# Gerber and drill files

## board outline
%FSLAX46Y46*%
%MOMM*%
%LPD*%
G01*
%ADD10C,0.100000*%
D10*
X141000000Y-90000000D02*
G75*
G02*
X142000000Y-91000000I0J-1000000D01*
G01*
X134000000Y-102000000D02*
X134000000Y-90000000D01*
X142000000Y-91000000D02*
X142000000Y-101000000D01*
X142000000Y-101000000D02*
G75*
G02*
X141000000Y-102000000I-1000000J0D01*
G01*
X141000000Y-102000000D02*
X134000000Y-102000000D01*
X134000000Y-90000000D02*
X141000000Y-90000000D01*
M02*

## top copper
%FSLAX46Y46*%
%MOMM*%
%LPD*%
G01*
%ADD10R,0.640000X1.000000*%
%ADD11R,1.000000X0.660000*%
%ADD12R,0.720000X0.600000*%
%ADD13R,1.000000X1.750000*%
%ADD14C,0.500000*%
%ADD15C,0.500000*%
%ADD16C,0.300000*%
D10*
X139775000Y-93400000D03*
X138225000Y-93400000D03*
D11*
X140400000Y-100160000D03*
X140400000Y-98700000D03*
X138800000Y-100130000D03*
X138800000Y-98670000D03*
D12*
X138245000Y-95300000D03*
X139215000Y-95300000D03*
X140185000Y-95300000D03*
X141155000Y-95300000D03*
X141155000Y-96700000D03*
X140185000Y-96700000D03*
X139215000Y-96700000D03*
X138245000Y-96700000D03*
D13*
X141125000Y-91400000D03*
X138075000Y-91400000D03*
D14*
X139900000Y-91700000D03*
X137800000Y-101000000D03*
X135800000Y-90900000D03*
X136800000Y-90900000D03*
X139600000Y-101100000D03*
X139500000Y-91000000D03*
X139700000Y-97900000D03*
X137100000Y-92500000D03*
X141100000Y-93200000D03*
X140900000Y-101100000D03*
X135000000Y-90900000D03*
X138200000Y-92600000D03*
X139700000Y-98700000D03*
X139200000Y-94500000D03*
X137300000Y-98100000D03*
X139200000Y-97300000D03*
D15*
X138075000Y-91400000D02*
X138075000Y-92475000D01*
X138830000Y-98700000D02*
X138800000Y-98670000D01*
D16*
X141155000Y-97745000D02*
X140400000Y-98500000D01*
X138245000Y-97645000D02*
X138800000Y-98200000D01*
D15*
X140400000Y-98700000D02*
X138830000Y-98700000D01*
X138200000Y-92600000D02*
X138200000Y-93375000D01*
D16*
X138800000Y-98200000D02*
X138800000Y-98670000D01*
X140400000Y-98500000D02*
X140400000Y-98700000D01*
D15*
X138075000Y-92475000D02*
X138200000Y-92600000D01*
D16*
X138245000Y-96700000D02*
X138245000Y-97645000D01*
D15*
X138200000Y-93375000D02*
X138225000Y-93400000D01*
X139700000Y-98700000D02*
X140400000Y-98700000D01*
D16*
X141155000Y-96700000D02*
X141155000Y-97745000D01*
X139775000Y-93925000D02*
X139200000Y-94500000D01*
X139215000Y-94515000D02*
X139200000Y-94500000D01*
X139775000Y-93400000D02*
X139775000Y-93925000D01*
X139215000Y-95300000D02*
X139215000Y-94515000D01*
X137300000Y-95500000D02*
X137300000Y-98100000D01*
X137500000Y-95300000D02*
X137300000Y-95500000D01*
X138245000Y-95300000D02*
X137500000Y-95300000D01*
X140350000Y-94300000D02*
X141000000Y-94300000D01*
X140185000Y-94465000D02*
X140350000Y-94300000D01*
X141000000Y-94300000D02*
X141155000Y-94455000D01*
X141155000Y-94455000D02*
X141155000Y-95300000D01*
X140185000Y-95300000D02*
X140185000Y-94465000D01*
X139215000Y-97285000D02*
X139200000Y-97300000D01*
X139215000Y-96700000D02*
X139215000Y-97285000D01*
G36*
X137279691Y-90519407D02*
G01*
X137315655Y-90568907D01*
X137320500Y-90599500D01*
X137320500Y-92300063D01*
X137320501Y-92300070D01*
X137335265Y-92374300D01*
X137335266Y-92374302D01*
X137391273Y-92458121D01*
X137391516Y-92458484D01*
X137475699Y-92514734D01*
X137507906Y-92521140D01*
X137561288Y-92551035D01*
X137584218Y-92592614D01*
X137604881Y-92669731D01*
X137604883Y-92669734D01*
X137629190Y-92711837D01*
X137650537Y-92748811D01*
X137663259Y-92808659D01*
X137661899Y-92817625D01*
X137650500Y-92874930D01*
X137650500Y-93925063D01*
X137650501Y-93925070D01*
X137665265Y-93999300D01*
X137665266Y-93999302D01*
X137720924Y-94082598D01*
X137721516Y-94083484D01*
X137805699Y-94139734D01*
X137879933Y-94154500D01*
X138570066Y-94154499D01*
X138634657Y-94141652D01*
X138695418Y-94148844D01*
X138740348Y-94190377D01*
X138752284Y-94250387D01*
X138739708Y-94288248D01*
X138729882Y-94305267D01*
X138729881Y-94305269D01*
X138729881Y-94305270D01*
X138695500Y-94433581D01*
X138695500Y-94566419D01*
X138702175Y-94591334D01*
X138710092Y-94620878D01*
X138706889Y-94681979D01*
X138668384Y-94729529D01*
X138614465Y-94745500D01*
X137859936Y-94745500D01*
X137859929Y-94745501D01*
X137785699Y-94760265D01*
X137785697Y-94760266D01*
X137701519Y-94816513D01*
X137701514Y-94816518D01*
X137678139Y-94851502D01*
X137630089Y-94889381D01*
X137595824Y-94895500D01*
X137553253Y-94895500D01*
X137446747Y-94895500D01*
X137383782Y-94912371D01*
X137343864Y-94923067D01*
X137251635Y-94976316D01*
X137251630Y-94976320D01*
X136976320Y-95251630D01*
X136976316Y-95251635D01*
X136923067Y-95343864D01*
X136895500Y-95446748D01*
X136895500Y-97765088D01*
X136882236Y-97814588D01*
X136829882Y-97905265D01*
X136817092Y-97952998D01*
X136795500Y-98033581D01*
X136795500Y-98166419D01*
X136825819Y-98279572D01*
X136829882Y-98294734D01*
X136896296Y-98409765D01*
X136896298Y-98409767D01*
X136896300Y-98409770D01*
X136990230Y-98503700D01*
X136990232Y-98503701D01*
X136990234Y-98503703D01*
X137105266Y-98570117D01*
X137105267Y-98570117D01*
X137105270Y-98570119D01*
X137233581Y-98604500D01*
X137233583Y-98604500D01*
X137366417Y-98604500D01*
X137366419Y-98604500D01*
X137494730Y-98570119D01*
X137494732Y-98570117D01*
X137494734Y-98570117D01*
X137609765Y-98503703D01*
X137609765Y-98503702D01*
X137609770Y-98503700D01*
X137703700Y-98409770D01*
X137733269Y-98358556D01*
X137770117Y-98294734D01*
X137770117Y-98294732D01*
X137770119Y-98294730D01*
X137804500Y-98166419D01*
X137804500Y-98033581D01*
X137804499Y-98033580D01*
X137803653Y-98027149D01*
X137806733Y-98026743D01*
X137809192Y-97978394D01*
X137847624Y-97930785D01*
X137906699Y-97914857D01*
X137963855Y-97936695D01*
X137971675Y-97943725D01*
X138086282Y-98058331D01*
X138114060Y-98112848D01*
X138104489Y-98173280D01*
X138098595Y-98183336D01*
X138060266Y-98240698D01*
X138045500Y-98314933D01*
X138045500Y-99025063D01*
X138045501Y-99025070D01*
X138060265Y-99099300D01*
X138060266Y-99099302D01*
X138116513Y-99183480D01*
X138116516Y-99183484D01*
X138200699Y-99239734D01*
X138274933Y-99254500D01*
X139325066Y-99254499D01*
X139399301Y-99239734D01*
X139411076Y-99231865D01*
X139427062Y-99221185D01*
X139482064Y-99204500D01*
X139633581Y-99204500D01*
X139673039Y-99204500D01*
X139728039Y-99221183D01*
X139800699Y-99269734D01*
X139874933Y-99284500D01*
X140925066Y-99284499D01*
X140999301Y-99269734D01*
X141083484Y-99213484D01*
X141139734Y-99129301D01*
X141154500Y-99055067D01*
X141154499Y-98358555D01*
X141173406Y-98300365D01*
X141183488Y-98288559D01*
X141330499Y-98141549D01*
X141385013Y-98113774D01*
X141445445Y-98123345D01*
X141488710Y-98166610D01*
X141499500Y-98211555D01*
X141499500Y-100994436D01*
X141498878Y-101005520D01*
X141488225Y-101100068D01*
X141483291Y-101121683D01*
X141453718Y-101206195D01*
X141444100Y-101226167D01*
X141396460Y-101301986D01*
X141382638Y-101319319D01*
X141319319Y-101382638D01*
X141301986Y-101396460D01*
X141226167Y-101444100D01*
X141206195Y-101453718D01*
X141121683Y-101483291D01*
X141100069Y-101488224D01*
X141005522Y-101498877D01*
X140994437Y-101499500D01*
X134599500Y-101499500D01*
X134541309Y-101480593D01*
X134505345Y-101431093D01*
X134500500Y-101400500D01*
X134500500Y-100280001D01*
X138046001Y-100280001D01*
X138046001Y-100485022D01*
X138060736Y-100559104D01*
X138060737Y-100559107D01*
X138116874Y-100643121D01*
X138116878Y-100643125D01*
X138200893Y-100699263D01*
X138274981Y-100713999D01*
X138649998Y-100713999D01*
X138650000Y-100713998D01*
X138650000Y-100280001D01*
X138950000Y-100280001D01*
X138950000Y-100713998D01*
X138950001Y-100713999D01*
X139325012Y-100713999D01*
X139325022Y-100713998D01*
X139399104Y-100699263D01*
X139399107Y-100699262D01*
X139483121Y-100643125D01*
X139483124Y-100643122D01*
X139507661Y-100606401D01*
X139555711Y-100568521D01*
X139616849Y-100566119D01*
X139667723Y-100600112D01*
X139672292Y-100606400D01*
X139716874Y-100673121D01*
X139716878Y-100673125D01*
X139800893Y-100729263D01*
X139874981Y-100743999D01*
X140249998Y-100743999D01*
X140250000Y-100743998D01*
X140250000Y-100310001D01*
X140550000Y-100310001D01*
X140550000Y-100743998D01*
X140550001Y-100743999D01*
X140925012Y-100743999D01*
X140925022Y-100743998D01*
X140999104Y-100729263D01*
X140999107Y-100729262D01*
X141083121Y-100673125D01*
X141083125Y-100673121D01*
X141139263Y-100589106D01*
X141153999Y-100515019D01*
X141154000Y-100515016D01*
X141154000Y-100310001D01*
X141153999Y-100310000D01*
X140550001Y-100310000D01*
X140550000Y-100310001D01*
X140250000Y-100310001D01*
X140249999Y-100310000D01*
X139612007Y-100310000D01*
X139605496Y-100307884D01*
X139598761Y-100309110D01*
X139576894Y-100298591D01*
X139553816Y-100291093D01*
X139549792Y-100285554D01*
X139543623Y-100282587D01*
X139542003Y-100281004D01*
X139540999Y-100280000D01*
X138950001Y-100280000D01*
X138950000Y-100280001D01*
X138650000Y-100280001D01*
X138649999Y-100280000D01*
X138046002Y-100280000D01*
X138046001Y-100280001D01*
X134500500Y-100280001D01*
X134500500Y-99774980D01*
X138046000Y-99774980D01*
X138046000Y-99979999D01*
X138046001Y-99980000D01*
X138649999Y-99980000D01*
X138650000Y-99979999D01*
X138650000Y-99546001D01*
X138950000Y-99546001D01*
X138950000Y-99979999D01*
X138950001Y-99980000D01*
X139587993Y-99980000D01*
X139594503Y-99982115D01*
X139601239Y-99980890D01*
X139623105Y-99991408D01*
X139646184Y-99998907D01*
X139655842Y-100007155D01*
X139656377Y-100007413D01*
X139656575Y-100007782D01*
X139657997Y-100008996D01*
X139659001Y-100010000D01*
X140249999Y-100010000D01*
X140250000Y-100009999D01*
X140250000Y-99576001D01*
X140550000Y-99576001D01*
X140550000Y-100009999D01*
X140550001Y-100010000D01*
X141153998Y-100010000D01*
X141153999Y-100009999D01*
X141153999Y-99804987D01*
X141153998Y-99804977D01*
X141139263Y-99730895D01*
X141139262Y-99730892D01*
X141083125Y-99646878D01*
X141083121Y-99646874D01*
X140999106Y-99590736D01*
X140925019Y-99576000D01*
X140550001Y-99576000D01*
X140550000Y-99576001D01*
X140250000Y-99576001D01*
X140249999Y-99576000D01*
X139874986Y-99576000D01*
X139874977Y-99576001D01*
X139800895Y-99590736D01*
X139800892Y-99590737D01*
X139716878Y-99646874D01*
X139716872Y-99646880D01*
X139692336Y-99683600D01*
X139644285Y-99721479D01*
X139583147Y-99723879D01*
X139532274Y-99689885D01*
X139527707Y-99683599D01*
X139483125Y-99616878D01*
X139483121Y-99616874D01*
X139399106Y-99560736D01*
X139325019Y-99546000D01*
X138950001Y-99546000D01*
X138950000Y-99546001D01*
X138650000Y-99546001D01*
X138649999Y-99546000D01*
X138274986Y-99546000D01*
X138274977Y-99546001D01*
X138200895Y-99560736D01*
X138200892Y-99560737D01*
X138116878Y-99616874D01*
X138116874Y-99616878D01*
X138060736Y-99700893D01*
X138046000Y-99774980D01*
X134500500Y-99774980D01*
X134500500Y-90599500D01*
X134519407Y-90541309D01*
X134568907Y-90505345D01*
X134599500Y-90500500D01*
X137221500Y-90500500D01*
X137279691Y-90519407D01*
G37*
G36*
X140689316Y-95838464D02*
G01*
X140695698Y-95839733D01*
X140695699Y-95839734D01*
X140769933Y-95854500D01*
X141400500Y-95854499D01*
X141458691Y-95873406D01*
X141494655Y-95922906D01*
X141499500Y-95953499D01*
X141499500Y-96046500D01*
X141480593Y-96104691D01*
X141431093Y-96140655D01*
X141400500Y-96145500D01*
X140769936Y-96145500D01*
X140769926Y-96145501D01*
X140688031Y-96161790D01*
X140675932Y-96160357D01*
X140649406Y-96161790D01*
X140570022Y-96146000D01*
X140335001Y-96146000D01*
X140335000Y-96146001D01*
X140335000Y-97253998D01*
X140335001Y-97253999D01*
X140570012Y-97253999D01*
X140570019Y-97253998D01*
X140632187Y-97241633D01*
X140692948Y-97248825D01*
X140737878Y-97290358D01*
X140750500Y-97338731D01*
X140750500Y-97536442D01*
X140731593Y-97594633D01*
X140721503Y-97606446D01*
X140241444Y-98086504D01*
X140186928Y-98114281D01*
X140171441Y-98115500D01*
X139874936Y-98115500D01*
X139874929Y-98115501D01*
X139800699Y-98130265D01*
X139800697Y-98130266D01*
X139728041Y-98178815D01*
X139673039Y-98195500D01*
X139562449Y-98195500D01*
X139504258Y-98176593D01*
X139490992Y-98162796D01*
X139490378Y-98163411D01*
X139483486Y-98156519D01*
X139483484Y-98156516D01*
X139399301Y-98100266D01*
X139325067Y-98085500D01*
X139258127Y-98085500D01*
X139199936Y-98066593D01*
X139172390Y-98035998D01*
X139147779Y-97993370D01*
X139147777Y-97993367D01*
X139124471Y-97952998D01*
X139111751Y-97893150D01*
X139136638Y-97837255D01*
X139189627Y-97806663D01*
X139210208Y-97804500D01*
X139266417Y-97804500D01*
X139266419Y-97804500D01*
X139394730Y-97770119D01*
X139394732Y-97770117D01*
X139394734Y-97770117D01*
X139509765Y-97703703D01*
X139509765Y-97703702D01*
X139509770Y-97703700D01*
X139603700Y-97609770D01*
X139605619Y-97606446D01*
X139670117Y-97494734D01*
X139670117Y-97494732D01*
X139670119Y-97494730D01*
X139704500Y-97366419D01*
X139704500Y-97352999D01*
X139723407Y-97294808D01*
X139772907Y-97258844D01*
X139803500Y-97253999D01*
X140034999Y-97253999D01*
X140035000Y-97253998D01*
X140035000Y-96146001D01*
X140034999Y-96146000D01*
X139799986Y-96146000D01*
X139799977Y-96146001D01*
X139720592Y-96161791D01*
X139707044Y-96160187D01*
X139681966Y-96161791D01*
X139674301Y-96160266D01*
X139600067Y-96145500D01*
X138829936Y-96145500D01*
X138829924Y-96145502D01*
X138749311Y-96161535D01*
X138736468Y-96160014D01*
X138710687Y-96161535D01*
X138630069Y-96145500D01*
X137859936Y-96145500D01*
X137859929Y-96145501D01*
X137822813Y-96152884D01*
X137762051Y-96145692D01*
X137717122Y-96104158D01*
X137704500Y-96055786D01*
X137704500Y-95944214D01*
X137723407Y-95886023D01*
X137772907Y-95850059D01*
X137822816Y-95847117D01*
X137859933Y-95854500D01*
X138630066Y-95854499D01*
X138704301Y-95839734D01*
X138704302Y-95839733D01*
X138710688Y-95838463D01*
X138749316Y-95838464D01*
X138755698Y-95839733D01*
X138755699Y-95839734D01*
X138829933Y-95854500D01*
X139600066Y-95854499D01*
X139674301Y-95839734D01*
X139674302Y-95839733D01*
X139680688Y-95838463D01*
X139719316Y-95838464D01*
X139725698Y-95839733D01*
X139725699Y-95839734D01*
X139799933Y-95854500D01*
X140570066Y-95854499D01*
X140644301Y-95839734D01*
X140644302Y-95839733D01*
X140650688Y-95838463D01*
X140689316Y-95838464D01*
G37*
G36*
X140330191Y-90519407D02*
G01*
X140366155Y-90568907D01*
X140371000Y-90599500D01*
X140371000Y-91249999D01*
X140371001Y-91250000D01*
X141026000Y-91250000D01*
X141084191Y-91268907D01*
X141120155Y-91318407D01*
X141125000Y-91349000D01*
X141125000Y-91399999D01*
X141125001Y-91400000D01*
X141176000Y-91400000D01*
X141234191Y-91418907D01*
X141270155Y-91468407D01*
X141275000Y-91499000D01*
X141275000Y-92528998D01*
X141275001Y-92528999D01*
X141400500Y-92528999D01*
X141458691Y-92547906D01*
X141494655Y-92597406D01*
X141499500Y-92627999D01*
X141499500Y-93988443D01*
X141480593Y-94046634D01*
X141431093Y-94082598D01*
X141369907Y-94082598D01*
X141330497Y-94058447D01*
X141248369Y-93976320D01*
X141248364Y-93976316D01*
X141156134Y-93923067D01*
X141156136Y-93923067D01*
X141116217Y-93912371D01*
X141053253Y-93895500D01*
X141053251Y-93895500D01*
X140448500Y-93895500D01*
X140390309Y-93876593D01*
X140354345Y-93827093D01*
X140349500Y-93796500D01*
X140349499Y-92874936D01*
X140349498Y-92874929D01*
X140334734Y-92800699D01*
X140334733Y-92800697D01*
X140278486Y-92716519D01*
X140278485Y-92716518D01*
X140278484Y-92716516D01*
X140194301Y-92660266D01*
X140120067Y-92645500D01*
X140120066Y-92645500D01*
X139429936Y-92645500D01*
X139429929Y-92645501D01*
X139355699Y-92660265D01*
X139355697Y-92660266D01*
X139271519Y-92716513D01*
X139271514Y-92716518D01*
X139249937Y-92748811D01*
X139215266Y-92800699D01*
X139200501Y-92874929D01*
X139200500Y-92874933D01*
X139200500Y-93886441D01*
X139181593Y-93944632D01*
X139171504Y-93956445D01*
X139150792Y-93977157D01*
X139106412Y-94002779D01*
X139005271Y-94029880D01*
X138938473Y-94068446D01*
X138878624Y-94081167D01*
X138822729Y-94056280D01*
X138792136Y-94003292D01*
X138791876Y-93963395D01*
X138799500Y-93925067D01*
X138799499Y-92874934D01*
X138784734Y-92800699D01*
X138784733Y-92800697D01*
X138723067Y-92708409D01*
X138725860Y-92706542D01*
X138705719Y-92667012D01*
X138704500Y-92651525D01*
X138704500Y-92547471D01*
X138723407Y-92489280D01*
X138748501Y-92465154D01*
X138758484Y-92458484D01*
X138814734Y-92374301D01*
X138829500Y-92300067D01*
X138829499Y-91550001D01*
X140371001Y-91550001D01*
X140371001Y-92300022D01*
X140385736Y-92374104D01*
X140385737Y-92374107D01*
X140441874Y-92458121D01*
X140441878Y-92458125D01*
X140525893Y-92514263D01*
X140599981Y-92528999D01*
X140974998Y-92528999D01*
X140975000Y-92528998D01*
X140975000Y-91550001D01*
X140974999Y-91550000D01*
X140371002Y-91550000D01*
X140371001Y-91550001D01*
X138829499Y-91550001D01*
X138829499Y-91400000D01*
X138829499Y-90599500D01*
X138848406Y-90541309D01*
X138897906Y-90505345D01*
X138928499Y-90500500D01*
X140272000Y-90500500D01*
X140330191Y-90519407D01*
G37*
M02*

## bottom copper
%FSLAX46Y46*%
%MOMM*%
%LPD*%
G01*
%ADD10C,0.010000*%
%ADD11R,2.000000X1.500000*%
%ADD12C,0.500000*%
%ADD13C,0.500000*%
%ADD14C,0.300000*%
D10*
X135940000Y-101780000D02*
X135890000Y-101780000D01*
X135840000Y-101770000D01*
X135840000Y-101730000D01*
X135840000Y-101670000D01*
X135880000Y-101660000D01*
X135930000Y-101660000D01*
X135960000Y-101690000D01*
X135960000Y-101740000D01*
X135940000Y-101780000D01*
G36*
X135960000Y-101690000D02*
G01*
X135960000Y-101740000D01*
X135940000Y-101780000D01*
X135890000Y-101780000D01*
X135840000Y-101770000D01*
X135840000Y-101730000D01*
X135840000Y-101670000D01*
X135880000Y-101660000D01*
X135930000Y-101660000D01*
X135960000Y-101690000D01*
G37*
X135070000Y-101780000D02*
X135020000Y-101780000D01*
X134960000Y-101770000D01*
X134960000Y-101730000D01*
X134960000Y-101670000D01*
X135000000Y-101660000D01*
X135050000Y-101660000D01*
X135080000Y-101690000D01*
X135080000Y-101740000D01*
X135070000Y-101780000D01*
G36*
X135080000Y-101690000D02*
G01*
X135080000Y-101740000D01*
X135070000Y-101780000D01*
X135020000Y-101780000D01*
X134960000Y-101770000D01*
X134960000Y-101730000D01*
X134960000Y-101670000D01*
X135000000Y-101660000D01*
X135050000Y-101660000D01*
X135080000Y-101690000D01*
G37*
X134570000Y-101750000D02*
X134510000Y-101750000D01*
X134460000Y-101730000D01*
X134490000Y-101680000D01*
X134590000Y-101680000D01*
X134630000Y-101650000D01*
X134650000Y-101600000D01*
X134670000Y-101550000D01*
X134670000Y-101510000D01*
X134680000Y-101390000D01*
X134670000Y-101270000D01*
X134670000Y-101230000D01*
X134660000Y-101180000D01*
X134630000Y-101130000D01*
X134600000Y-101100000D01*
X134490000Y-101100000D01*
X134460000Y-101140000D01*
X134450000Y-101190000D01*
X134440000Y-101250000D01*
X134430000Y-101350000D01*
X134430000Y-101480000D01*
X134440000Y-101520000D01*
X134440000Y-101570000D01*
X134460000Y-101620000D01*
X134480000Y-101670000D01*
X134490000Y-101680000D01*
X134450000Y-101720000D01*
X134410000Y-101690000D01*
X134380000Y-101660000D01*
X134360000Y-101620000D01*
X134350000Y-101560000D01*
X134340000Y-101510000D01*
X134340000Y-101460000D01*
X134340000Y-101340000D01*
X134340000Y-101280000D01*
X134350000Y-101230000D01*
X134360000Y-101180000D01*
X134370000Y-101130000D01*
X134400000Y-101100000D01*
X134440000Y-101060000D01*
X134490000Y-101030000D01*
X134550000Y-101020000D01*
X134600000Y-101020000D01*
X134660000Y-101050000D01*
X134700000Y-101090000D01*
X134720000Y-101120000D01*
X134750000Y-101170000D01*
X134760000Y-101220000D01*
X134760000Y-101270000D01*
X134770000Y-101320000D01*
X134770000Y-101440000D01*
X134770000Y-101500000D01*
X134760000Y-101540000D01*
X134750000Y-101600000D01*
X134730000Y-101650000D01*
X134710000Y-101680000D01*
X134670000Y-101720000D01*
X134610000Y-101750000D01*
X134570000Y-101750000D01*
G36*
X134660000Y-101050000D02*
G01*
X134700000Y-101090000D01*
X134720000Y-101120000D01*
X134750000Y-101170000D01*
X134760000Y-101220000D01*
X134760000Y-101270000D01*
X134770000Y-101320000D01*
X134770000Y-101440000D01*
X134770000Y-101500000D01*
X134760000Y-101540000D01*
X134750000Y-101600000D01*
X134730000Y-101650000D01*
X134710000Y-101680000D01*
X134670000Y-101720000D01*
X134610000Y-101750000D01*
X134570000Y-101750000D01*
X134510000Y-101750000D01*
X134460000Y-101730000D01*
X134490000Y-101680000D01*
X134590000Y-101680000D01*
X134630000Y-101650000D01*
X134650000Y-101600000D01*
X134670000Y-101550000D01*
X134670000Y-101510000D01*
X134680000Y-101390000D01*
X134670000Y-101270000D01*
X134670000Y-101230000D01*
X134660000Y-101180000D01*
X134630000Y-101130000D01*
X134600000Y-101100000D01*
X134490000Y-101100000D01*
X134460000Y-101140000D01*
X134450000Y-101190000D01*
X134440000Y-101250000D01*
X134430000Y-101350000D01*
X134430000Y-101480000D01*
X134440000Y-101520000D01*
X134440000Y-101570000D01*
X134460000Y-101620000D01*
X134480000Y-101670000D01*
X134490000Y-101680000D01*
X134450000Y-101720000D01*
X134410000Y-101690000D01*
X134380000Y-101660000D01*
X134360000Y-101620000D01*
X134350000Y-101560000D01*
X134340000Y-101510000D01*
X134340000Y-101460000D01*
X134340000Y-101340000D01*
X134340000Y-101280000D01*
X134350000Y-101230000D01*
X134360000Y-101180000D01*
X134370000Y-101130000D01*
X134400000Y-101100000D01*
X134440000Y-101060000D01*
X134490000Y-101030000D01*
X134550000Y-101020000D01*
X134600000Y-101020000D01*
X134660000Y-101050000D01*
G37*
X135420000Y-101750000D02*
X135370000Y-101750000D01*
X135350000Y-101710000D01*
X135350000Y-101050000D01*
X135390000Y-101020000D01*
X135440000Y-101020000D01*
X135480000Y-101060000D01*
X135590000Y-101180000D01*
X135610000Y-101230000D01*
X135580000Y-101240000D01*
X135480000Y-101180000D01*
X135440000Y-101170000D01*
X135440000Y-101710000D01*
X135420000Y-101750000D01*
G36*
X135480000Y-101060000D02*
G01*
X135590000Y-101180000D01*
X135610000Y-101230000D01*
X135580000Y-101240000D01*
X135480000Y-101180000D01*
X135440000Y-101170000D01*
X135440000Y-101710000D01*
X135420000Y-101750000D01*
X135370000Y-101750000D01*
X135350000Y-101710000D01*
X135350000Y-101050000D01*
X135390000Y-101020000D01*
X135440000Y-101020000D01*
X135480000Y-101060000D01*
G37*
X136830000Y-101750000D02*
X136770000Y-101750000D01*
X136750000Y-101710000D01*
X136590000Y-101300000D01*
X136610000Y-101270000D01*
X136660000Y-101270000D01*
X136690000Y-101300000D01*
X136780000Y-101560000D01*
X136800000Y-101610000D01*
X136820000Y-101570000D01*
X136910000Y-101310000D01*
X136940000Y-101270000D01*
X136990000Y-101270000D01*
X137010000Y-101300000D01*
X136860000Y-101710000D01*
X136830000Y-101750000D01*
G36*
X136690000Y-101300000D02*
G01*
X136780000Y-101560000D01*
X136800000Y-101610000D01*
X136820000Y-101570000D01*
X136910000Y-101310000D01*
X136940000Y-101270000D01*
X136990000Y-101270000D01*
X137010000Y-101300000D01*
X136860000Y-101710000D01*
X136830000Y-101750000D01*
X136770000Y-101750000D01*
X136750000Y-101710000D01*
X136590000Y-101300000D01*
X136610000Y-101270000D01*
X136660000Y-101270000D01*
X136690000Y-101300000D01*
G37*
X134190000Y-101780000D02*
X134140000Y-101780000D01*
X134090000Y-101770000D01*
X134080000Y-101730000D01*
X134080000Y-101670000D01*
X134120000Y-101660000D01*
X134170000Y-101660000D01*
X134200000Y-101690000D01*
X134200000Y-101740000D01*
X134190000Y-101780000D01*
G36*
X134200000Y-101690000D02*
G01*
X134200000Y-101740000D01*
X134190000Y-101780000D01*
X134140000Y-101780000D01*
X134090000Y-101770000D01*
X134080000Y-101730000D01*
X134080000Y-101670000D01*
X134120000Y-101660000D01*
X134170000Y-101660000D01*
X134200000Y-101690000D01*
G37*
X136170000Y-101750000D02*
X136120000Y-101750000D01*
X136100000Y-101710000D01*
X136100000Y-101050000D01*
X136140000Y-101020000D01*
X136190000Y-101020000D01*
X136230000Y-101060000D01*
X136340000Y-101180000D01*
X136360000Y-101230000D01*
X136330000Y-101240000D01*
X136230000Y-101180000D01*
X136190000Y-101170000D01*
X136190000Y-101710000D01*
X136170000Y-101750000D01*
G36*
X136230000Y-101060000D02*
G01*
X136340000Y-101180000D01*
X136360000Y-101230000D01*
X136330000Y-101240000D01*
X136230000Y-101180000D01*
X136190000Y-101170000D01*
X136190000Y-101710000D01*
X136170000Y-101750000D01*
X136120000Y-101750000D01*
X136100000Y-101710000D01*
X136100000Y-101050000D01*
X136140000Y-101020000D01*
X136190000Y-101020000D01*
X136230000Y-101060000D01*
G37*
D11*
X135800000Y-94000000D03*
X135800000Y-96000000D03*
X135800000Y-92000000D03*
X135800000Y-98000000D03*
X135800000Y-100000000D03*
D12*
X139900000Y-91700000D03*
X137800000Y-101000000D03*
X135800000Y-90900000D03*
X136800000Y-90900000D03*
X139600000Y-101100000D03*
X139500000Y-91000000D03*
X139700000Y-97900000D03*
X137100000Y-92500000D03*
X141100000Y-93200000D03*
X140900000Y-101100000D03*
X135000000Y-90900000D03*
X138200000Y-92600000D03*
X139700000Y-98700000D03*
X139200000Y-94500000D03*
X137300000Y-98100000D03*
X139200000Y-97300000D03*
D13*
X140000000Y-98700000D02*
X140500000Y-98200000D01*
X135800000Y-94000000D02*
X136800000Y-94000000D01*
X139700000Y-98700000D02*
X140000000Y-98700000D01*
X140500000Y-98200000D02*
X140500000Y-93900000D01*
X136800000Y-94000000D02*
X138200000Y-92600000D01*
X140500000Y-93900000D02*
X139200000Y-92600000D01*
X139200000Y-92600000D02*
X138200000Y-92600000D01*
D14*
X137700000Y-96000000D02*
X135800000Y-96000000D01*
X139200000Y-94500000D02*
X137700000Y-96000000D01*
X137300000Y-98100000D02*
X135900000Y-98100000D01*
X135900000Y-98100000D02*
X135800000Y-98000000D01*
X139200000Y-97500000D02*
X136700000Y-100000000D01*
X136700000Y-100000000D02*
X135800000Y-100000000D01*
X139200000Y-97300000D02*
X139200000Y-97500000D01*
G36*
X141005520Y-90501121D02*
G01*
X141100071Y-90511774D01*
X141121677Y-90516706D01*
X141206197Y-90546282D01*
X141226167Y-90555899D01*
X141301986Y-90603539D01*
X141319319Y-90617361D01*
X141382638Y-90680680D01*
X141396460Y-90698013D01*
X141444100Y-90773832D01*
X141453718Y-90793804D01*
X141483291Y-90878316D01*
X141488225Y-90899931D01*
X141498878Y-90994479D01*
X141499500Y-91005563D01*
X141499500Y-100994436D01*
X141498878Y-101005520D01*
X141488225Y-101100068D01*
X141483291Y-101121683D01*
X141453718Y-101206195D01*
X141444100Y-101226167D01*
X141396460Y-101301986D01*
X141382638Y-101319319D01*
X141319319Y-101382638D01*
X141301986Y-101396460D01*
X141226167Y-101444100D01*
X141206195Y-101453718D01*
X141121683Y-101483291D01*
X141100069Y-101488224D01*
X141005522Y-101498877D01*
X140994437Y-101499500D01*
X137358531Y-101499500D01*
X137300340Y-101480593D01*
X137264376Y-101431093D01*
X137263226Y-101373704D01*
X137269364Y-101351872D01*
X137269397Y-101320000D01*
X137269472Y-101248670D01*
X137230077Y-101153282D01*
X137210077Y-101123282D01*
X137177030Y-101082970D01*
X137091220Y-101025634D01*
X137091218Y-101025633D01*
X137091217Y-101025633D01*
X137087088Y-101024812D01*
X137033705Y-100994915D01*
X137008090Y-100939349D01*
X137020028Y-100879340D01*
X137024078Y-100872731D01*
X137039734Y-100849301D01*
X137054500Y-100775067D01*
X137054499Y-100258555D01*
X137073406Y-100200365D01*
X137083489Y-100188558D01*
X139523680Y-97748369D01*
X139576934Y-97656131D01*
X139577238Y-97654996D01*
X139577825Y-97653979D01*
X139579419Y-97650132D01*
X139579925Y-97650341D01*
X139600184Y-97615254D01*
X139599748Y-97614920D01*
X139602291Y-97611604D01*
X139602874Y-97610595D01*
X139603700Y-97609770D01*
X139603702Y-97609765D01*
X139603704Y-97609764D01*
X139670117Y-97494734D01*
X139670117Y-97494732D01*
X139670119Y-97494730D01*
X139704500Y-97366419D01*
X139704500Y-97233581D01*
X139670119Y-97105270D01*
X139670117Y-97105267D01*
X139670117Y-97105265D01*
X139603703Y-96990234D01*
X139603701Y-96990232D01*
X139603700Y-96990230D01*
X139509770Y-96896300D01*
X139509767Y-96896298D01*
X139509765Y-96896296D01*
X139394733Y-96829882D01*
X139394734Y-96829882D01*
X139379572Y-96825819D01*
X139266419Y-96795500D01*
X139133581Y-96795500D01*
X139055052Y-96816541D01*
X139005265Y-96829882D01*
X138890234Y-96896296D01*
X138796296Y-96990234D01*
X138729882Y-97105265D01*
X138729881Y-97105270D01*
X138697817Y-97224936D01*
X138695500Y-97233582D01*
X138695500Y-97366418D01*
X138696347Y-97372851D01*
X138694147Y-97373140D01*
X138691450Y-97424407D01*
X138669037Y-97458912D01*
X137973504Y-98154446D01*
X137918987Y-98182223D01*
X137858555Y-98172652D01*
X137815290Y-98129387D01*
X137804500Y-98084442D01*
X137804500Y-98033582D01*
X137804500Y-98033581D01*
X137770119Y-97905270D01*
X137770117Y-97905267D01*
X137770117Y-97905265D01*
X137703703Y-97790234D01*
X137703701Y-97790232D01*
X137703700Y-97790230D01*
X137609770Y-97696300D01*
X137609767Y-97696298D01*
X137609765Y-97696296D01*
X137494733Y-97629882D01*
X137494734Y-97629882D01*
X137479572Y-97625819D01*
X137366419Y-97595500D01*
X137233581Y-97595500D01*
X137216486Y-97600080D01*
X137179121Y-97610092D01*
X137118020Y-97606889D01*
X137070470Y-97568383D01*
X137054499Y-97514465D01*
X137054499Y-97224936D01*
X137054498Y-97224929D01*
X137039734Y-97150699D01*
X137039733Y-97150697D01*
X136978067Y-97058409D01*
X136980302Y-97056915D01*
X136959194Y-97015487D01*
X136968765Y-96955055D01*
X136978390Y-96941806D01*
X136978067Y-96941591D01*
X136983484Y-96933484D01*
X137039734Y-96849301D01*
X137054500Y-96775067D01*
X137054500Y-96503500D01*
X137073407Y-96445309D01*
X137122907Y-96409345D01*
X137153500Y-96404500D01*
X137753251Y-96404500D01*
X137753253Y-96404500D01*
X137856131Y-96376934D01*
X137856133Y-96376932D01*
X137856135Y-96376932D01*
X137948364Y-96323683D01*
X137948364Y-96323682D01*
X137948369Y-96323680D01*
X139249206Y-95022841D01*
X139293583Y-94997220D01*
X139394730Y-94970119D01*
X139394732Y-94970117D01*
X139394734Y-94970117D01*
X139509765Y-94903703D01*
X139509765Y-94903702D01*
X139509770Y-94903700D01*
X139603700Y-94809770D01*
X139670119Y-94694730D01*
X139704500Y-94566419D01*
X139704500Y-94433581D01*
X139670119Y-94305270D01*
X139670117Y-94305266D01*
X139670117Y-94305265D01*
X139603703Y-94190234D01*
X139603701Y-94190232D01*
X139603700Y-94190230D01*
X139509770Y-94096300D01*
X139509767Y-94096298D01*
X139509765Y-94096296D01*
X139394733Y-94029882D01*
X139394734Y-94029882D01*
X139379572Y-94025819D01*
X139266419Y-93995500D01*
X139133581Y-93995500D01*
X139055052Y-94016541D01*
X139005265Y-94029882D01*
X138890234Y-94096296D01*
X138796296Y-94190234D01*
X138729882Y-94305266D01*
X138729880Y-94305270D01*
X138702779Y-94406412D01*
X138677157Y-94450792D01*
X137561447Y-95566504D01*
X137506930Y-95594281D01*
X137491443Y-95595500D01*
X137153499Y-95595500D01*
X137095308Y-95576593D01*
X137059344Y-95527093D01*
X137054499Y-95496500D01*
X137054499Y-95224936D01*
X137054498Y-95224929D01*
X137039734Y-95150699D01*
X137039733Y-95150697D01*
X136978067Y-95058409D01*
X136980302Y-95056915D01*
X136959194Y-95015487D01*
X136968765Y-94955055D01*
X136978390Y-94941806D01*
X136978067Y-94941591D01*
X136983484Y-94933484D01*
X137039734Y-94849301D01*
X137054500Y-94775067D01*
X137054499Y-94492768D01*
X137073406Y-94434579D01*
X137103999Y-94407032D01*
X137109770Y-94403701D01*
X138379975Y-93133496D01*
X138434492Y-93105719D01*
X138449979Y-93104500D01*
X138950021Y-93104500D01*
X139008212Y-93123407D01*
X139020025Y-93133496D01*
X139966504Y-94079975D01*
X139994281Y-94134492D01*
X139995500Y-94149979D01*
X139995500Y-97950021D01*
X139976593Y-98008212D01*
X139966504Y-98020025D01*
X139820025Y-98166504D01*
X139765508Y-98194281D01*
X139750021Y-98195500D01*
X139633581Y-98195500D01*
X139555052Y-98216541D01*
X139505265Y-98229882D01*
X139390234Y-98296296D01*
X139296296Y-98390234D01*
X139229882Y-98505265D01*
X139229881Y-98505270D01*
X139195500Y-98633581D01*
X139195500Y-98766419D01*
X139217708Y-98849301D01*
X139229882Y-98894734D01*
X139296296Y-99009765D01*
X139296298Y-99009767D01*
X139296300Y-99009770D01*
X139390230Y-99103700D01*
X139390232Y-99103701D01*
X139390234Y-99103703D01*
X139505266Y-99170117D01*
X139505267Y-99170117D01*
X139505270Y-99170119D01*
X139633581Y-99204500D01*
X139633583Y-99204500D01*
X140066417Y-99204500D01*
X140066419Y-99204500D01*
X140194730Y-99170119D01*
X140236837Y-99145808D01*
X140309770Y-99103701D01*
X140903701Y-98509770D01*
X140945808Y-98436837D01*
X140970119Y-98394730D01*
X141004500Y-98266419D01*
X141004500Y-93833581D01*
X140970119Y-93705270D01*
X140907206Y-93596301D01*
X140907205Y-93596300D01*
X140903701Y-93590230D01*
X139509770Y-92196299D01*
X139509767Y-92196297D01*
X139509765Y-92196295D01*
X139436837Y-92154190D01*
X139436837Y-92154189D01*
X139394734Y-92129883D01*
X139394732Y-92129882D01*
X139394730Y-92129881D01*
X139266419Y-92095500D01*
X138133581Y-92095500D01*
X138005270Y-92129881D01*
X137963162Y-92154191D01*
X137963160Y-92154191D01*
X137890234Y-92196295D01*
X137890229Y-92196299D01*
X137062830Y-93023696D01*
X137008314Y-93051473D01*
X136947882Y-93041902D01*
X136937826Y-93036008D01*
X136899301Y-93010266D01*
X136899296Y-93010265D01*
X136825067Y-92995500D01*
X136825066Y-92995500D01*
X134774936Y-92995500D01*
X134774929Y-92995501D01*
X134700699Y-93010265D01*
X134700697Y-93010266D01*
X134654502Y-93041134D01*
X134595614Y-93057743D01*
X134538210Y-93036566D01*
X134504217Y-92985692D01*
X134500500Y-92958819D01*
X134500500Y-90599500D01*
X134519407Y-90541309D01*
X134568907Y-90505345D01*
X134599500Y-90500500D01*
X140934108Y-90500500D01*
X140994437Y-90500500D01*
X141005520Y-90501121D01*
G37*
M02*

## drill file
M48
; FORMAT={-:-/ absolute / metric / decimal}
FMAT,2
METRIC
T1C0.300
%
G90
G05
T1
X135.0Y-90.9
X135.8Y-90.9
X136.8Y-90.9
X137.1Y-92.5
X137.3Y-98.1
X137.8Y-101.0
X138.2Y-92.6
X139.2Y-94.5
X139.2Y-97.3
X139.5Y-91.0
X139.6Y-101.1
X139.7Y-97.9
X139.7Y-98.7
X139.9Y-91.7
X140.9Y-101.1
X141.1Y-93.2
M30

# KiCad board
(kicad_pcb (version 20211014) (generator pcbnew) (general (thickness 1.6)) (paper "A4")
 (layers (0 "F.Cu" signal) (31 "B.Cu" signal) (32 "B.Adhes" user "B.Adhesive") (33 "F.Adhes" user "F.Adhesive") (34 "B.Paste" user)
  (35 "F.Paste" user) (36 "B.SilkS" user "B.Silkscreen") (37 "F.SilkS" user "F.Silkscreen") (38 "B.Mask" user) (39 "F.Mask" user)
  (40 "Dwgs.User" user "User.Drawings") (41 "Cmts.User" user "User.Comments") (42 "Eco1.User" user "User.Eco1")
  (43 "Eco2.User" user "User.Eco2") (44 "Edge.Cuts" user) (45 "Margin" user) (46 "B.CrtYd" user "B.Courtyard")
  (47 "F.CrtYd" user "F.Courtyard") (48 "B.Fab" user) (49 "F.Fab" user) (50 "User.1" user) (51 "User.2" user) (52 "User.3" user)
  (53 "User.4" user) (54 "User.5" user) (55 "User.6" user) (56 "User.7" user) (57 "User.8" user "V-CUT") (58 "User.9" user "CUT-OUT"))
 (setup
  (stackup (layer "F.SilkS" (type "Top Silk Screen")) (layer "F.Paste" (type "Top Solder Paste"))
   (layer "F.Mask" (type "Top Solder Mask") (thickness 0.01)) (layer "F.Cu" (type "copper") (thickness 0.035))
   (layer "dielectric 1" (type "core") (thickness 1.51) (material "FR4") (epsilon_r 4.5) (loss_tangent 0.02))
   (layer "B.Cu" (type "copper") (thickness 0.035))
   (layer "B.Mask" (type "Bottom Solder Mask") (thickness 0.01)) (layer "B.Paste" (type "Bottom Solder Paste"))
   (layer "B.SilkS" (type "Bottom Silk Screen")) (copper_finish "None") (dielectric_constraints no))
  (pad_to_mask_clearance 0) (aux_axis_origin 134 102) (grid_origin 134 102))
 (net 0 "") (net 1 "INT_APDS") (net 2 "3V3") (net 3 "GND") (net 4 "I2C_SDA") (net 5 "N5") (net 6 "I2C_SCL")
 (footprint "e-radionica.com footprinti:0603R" (layer "F.Cu") (at 139 93.4 180)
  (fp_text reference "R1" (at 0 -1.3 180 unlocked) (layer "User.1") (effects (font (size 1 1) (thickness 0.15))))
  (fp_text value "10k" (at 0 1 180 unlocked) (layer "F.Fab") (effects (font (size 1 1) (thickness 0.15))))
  (pad "1" smd rect locked (at -0.775 0 270) (size 1 0.64) (layers "F.Cu" "F.Paste" "F.Mask") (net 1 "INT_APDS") (solder_mask_margin 0.1))
  (pad "2" smd rect locked (at 0.775 0 270) (size 1 0.64) (layers "F.Cu" "F.Paste" "F.Mask") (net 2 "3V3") (solder_mask_margin 0.1)))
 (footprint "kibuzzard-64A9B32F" (layer "F.Cu") (at 135 96 -90)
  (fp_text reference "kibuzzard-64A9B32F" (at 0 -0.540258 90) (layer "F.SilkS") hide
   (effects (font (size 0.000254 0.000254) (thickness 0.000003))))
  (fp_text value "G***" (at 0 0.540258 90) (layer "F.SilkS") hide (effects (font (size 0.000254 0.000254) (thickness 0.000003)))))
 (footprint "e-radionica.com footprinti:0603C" (layer "F.Cu") (at 140.4 99.43 90)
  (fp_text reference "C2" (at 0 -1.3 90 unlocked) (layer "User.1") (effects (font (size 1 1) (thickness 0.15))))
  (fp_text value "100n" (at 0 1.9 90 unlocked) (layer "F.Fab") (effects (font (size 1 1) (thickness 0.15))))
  (pad "1" smd rect locked (at -0.73 0 90) (size 0.66 1) (layers "F.Cu" "F.Paste" "F.Mask") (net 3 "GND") (solder_mask_margin 0.1))
  (pad "2" smd rect locked (at 0.73 0 90) (size 0.66 1) (layers "F.Cu" "F.Paste" "F.Mask") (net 2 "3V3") (solder_mask_margin 0.1)))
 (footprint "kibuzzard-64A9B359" (layer "F.Cu") (at 136.5 96 -90)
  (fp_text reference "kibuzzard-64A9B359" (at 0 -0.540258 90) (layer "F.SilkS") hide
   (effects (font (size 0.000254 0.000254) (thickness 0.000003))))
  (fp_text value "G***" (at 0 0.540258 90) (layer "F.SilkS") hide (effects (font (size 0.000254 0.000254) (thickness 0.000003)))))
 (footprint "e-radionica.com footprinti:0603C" (layer "F.Cu") (at 138.8 99.4 90)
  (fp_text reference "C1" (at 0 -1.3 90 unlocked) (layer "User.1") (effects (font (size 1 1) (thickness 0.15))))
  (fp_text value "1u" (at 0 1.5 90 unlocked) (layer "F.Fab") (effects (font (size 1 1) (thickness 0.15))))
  (pad "1" smd rect locked (at -0.73 0 90) (size 0.66 1) (layers "F.Cu" "F.Paste" "F.Mask") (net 3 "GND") (solder_mask_margin 0.1))
  (pad "2" smd rect locked (at 0.73 0 90) (size 0.66 1) (layers "F.Cu" "F.Paste" "F.Mask") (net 2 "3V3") (solder_mask_margin 0.1)))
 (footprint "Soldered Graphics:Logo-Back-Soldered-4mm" (layer "F.Cu") (at 139.5 96 90)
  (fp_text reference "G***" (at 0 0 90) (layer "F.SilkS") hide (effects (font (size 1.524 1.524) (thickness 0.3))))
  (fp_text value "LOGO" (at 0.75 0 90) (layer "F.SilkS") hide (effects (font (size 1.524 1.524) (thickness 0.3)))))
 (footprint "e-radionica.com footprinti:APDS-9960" (layer "F.Cu") (at 139.7 96 90)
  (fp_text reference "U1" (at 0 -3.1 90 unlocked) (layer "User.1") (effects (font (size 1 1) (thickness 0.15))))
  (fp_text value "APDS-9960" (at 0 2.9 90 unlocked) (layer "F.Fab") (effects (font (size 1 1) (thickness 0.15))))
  (pad "1" smd rect (at 0.7 -1.455 90) (size 0.6 0.72) (layers "F.Cu" "F.Paste" "F.Mask") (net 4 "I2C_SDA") (solder_mask_margin 0.1))
  (pad "2" smd rect (at 0.7 -0.485 90) (size 0.6 0.72) (layers "F.Cu" "F.Paste" "F.Mask") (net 1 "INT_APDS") (solder_mask_margin 0.1))
  (pad "3" smd rect (at 0.7 0.485 90) (size 0.6 0.72) (layers "F.Cu" "F.Paste" "F.Mask") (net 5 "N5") (solder_mask_margin 0.1))
  (pad "4" smd rect (at 0.7 1.455 90) (size 0.6 0.72) (layers "F.Cu" "F.Paste" "F.Mask") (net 5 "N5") (solder_mask_margin 0.1))
  (pad "5" smd rect (at -0.7 1.455 90) (size 0.6 0.72) (layers "F.Cu" "F.Paste" "F.Mask") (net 2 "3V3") (solder_mask_margin 0.1))
  (pad "6" smd rect (at -0.7 0.485 90) (size 0.6 0.72) (layers "F.Cu" "F.Paste" "F.Mask") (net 3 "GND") (solder_mask_margin 0.1))
  (pad "7" smd rect (at -0.7 -0.485 90) (size 0.6 0.72) (layers "F.Cu" "F.Paste" "F.Mask") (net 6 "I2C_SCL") (solder_mask_margin 0.1))
  (pad "8" smd rect (at -0.7 -1.455 90) (size 0.6 0.72) (layers "F.Cu" "F.Paste" "F.Mask") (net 2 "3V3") (solder_mask_margin 0.1)))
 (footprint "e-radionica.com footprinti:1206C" (layer "F.Cu") (at 139.6 91.4 180)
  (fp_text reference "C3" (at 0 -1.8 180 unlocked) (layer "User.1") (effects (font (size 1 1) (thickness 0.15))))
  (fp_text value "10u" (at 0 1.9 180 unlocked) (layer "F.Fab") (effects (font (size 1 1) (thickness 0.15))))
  (pad "1" smd rect locked (at -1.525 0 270) (size 1.75 1) (layers "F.Cu" "F.Paste" "F.Mask") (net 3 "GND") (solder_mask_margin 0.1))
  (pad "2" smd rect locked (at 1.525 0 270) (size 1.75 1) (layers "F.Cu" "F.Paste" "F.Mask") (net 2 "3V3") (solder_mask_margin 0.1)))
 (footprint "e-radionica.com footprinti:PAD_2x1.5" (layer "B.Cu") (at 135.8 94 180)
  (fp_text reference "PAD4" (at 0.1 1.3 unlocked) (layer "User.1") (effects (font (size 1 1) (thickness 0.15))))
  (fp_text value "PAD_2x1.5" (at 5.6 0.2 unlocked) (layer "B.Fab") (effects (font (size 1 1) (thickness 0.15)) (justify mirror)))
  (pad "1" smd rect (at 0 0 180) (size 2 1.5) (layers "B.Cu" "B.Paste" "B.Mask") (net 2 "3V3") (solder_mask_margin 0.1)))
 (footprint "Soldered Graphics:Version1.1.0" (layer "B.Cu") (at 135.5 101.4 180)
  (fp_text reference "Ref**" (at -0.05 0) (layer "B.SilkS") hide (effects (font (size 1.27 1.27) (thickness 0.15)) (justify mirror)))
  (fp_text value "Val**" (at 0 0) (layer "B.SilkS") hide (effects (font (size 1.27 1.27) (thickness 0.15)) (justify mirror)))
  (fp_poly
   (pts (xy -0.44 -0.38) (xy -0.39 -0.38) (xy -0.34 -0.37) (xy -0.34 -0.33) (xy -0.34 -0.27) (xy -0.38 -0.26) (xy -0.43 -0.26)
    (xy -0.46 -0.29) (xy -0.46 -0.34) (xy -0.44 -0.38))
   (layer "B.Cu") (width 0.01) (fill solid))
  (fp_poly
   (pts (xy 0.43 -0.38) (xy 0.48 -0.38) (xy 0.54 -0.37) (xy 0.54 -0.33) (xy 0.54 -0.27) (xy 0.5 -0.26) (xy 0.45 -0.26) (xy 0.42 -0.29)
    (xy 0.42 -0.34) (xy 0.43 -0.38))
   (layer "B.Cu") (width 0.01) (fill solid))
  (fp_poly
   (pts (xy 0.93 -0.35) (xy 0.99 -0.35) (xy 1.04 -0.33) (xy 1.01 -0.28) (xy 0.91 -0.28) (xy 0.87 -0.25) (xy 0.85 -0.2) (xy 0.83 -0.15)
    (xy 0.83 -0.11) (xy 0.82 0.01) (xy 0.83 0.13) (xy 0.83 0.17) (xy 0.84 0.22) (xy 0.87 0.27) (xy 0.9 0.3) (xy 1.01 0.3) (xy 1.04 0.26)
    (xy 1.05 0.21) (xy 1.06 0.15) (xy 1.07 0.05) (xy 1.07 -0.08) (xy 1.06 -0.12) (xy 1.06 -0.17) (xy 1.04 -0.22) (xy 1.02 -0.27)
    (xy 1.01 -0.28) (xy 1.05 -0.32) (xy 1.09 -0.29) (xy 1.12 -0.26) (xy 1.14 -0.22) (xy 1.15 -0.16) (xy 1.16 -0.11) (xy 1.16 -0.06)
    (xy 1.16 0.06) (xy 1.16 0.12) (xy 1.15 0.17) (xy 1.14 0.22) (xy 1.13 0.27) (xy 1.1 0.3) (xy 1.06 0.34) (xy 1.01 0.37) (xy 0.95 0.38)
    (xy 0.9 0.38) (xy 0.84 0.35) (xy 0.8 0.31) (xy 0.78 0.28) (xy 0.75 0.23) (xy 0.74 0.18) (xy 0.74 0.13) (xy 0.73 0.08) (xy 0.73 -0.04)
    (xy 0.73 -0.1) (xy 0.74 -0.14) (xy 0.75 -0.2) (xy 0.77 -0.25) (xy 0.79 -0.28) (xy 0.83 -0.32) (xy 0.89 -0.35) (xy 0.93 -0.35))
   (layer "B.Cu") (width 0.01) (fill solid))
  (fp_poly
   (pts (xy 0.08 -0.35) (xy 0.13 -0.35) (xy 0.15 -0.31) (xy 0.15 0.35) (xy 0.11 0.38) (xy 0.06 0.38) (xy 0.02 0.34) (xy -0.09 0.22)
    (xy -0.11 0.17) (xy -0.08 0.16) (xy 0.02 0.22) (xy 0.06 0.23) (xy 0.06 -0.31) (xy 0.08 -0.35))
   (layer "B.Cu") (width 0.01) (fill solid))
  (fp_poly
   (pts (xy -1.33 -0.35) (xy -1.27 -0.35) (xy -1.25 -0.31) (xy -1.09 0.1) (xy -1.11 0.13) (xy -1.16 0.13) (xy -1.19 0.1) (xy -1.28 -0.16)
    (xy -1.3 -0.21) (xy -1.32 -0.17) (xy -1.41 0.09) (xy -1.44 0.13) (xy -1.49 0.13) (xy -1.51 0.1) (xy -1.36 -0.31) (xy -1.33 -0.35))
   (layer "B.Cu") (width 0.01) (fill solid))
  (fp_poly
   (pts (xy 1.31 -0.38) (xy 1.36 -0.38) (xy 1.41 -0.37) (xy 1.42 -0.33) (xy 1.42 -0.27) (xy 1.38 -0.26) (xy 1.33 -0.26) (xy 1.3 -0.29)
    (xy 1.3 -0.34) (xy 1.31 -0.38))
   (layer "B.Cu") (width 0.01) (fill solid))
  (fp_poly
   (pts (xy -0.67 -0.35) (xy -0.62 -0.35) (xy -0.6 -0.31) (xy -0.6 0.35) (xy -0.64 0.38) (xy -0.69 0.38) (xy -0.73 0.34) (xy -0.84 0.22)
    (xy -0.86 0.17) (xy -0.83 0.16) (xy -0.73 0.22) (xy -0.69 0.23) (xy -0.69 -0.31) (xy -0.67 -0.35))
   (layer "B.Cu") (width 0.01) (fill solid)))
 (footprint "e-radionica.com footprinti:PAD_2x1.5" (layer "B.Cu") (at 135.8 96 180)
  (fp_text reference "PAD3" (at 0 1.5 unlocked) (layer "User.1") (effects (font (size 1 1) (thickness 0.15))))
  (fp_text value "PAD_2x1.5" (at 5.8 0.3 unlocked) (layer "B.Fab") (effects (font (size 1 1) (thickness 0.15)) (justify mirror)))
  (pad "1" smd rect (at 0 0 180) (size 2 1.5) (layers "B.Cu" "B.Paste" "B.Mask") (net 1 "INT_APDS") (solder_mask_margin 0.1)))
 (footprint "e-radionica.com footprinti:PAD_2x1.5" (layer "B.Cu") (at 135.8 92 180)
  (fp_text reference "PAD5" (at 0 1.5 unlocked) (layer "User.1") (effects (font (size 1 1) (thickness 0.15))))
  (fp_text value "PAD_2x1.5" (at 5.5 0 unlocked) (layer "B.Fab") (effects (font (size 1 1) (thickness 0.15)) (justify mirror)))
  (pad "1" smd rect (at 0 0 180) (size 2 1.5) (layers "B.Cu" "B.Paste" "B.Mask") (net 3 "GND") (solder_mask_margin 0.1) (zone_connect 2)))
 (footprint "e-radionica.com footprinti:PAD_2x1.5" (layer "B.Cu") (at 135.8 98 180)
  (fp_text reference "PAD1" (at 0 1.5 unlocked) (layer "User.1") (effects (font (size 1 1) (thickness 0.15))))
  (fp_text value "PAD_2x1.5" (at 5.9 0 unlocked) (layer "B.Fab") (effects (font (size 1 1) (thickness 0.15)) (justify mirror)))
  (pad "1" smd rect (at 0 0 180) (size 2 1.5) (layers "B.Cu" "B.Paste" "B.Mask") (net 4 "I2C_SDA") (solder_mask_margin 0.1)))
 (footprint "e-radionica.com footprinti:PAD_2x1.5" (layer "B.Cu") (at 135.8 100 180)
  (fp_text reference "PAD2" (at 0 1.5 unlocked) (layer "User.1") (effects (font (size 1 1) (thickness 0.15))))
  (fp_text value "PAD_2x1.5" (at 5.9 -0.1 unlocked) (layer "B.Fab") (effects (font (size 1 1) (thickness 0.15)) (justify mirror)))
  (pad "1" smd rect (at 0 0 180) (size 2 1.5) (layers "B.Cu" "B.Paste" "B.Mask") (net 6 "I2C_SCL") (solder_mask_margin 0.1)))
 (gr_arc (start 141 90) (mid 141.707107 90.292893) (end 142 91) (layer "Edge.Cuts") (width 0.1))
 (gr_line (start 134 102) (end 134 90) (layer "Edge.Cuts") (width 0.1))
 (gr_line (start 142 91) (end 142 101) (layer "Edge.Cuts") (width 0.1))
 (gr_arc (start 142 101) (mid 141.707107 101.707107) (end 141 102) (layer "Edge.Cuts") (width 0.1))
 (gr_line (start 141 102) (end 134 102) (layer "Edge.Cuts") (width 0.1))
 (gr_line (start 134 90) (end 141 90) (layer "Edge.Cuts") (width 0.1))
 (via (at 139.9 91.7) (size 0.5) (drill 0.3) (layers "F.Cu" "B.Cu") (free) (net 3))
 (via (at 137.8 101) (size 0.5) (drill 0.3) (layers "F.Cu" "B.Cu") (free) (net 3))
 (via (at 135.8 90.9) (size 0.5) (drill 0.3) (layers "F.Cu" "B.Cu") (free) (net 3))
 (via (at 136.8 90.9) (size 0.5) (drill 0.3) (layers "F.Cu" "B.Cu") (free) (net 3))
 (via (at 139.6 101.1) (size 0.5) (drill 0.3) (layers "F.Cu" "B.Cu") (free) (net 3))
 (via (at 139.5 91) (size 0.5) (drill 0.3) (layers "F.Cu" "B.Cu") (free) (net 3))
 (via (at 139.7 97.9) (size 0.5) (drill 0.3) (layers "F.Cu" "B.Cu") (free) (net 3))
 (via (at 137.1 92.5) (size 0.5) (drill 0.3) (layers "F.Cu" "B.Cu") (free) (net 3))
 (via (at 141.1 93.2) (size 0.5) (drill 0.3) (layers "F.Cu" "B.Cu") (free) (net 3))
 (via (at 140.9 101.1) (size 0.5) (drill 0.3) (layers "F.Cu" "B.Cu") (free) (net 3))
 (via (at 135 90.9) (size 0.5) (drill 0.3) (layers "F.Cu" "B.Cu") (free) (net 3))
 (segment (start 138.075 91.4) (end 138.075 92.475) (width 0.5) (layer "F.Cu") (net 2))
 (segment (start 138.83 98.7) (end 138.8 98.67) (width 0.5) (layer "F.Cu") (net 2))
 (segment (start 141.155 97.745) (end 140.4 98.5) (width 0.3) (layer "F.Cu") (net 2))
 (segment (start 138.245 97.645) (end 138.8 98.2) (width 0.3) (layer "F.Cu") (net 2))
 (segment (start 140.4 98.7) (end 138.83 98.7) (width 0.5) (layer "F.Cu") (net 2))
 (segment (start 138.2 92.6) (end 138.2 93.375) (width 0.5) (layer "F.Cu") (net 2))
 (segment (start 138.8 98.2) (end 138.8 98.67) (width 0.3) (layer "F.Cu") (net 2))
 (segment (start 140.4 98.5) (end 140.4 98.7) (width 0.3) (layer "F.Cu") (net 2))
 (segment (start 138.075 92.475) (end 138.2 92.6) (width 0.5) (layer "F.Cu") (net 2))
 (segment (start 138.245 96.7) (end 138.245 97.645) (width 0.3) (layer "F.Cu") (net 2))
 (segment (start 138.2 93.375) (end 138.225 93.4) (width 0.5) (layer "F.Cu") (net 2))
 (segment (start 139.7 98.7) (end 140.4 98.7) (width 0.5) (layer "F.Cu") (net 2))
 (segment (start 141.155 96.7) (end 141.155 97.745) (width 0.3) (layer "F.Cu") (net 2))
 (via (at 138.2 92.6) (size 0.5) (drill 0.3) (layers "F.Cu" "B.Cu") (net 2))
 (via (at 139.7 98.7) (size 0.5) (drill 0.3) (layers "F.Cu" "B.Cu") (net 2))
 (segment (start 140 98.7) (end 140.5 98.2) (width 0.5) (layer "B.Cu") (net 2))
 (segment (start 135.8 94) (end 136.8 94) (width 0.5) (layer "B.Cu") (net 2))
 (segment (start 139.7 98.7) (end 140 98.7) (width 0.5) (layer "B.Cu") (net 2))
 (segment (start 140.5 98.2) (end 140.5 93.9) (width 0.5) (layer "B.Cu") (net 2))
 (segment (start 136.8 94) (end 138.2 92.6) (width 0.5) (layer "B.Cu") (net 2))
 (segment (start 140.5 93.9) (end 139.2 92.6) (width 0.5) (layer "B.Cu") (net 2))
 (segment (start 139.2 92.6) (end 138.2 92.6) (width 0.5) (layer "B.Cu") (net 2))
 (segment (start 139.775 93.925) (end 139.2 94.5) (width 0.3) (layer "F.Cu") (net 1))
 (segment (start 139.215 94.515) (end 139.2 94.5) (width 0.3) (layer "F.Cu") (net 1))
 (segment (start 139.775 93.4) (end 139.775 93.925) (width 0.3) (layer "F.Cu") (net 1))
 (segment (start 139.215 95.3) (end 139.215 94.515) (width 0.3) (layer "F.Cu") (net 1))
 (via (at 139.2 94.5) (size 0.5) (drill 0.3) (layers "F.Cu" "B.Cu") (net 1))
 (segment (start 137.7 96) (end 135.8 96) (width 0.3) (layer "B.Cu") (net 1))
 (segment (start 139.2 94.5) (end 137.7 96) (width 0.3) (layer "B.Cu") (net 1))
 (segment (start 137.3 95.5) (end 137.3 98.1) (width 0.3) (layer "F.Cu") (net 4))
 (segment (start 137.5 95.3) (end 137.3 95.5) (width 0.3) (layer "F.Cu") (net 4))
 (segment (start 138.245 95.3) (end 137.5 95.3) (width 0.3) (layer "F.Cu") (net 4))
 (via (at 137.3 98.1) (size 0.5) (drill 0.3) (layers "F.Cu" "B.Cu") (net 4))
 (segment (start 137.3 98.1) (end 135.9 98.1) (width 0.3) (layer "B.Cu") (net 4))
 (segment (start 135.9 98.1) (end 135.8 98) (width 0.3) (layer "B.Cu") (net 4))
 (segment (start 140.35 94.3) (end 141 94.3) (width 0.3) (layer "F.Cu") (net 5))
 (segment (start 140.185 94.465) (end 140.35 94.3) (width 0.3) (layer "F.Cu") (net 5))
 (segment (start 141 94.3) (end 141.155 94.455) (width 0.3) (layer "F.Cu") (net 5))
 (segment (start 141.155 94.455) (end 141.155 95.3) (width 0.3) (layer "F.Cu") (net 5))
 (segment (start 140.185 95.3) (end 140.185 94.465) (width 0.3) (layer "F.Cu") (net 5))
 (segment (start 139.215 97.285) (end 139.2 97.3) (width 0.3) (layer "F.Cu") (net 6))
 (segment (start 139.215 96.7) (end 139.215 97.285) (width 0.3) (layer "F.Cu") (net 6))
 (via (at 139.2 97.3) (size 0.5) (drill 0.3) (layers "F.Cu" "B.Cu") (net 6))
 (segment (start 139.2 97.5) (end 136.7 100) (width 0.3) (layer "B.Cu") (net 6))
 (segment (start 136.7 100) (end 135.8 100) (width 0.3) (layer "B.Cu") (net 6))
 (segment (start 139.2 97.3) (end 139.2 97.5) (width 0.3) (layer "B.Cu") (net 6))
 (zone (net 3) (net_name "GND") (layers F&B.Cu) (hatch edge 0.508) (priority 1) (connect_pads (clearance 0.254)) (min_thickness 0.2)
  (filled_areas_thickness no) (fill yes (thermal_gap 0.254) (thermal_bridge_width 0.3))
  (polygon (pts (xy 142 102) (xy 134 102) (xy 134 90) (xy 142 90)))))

